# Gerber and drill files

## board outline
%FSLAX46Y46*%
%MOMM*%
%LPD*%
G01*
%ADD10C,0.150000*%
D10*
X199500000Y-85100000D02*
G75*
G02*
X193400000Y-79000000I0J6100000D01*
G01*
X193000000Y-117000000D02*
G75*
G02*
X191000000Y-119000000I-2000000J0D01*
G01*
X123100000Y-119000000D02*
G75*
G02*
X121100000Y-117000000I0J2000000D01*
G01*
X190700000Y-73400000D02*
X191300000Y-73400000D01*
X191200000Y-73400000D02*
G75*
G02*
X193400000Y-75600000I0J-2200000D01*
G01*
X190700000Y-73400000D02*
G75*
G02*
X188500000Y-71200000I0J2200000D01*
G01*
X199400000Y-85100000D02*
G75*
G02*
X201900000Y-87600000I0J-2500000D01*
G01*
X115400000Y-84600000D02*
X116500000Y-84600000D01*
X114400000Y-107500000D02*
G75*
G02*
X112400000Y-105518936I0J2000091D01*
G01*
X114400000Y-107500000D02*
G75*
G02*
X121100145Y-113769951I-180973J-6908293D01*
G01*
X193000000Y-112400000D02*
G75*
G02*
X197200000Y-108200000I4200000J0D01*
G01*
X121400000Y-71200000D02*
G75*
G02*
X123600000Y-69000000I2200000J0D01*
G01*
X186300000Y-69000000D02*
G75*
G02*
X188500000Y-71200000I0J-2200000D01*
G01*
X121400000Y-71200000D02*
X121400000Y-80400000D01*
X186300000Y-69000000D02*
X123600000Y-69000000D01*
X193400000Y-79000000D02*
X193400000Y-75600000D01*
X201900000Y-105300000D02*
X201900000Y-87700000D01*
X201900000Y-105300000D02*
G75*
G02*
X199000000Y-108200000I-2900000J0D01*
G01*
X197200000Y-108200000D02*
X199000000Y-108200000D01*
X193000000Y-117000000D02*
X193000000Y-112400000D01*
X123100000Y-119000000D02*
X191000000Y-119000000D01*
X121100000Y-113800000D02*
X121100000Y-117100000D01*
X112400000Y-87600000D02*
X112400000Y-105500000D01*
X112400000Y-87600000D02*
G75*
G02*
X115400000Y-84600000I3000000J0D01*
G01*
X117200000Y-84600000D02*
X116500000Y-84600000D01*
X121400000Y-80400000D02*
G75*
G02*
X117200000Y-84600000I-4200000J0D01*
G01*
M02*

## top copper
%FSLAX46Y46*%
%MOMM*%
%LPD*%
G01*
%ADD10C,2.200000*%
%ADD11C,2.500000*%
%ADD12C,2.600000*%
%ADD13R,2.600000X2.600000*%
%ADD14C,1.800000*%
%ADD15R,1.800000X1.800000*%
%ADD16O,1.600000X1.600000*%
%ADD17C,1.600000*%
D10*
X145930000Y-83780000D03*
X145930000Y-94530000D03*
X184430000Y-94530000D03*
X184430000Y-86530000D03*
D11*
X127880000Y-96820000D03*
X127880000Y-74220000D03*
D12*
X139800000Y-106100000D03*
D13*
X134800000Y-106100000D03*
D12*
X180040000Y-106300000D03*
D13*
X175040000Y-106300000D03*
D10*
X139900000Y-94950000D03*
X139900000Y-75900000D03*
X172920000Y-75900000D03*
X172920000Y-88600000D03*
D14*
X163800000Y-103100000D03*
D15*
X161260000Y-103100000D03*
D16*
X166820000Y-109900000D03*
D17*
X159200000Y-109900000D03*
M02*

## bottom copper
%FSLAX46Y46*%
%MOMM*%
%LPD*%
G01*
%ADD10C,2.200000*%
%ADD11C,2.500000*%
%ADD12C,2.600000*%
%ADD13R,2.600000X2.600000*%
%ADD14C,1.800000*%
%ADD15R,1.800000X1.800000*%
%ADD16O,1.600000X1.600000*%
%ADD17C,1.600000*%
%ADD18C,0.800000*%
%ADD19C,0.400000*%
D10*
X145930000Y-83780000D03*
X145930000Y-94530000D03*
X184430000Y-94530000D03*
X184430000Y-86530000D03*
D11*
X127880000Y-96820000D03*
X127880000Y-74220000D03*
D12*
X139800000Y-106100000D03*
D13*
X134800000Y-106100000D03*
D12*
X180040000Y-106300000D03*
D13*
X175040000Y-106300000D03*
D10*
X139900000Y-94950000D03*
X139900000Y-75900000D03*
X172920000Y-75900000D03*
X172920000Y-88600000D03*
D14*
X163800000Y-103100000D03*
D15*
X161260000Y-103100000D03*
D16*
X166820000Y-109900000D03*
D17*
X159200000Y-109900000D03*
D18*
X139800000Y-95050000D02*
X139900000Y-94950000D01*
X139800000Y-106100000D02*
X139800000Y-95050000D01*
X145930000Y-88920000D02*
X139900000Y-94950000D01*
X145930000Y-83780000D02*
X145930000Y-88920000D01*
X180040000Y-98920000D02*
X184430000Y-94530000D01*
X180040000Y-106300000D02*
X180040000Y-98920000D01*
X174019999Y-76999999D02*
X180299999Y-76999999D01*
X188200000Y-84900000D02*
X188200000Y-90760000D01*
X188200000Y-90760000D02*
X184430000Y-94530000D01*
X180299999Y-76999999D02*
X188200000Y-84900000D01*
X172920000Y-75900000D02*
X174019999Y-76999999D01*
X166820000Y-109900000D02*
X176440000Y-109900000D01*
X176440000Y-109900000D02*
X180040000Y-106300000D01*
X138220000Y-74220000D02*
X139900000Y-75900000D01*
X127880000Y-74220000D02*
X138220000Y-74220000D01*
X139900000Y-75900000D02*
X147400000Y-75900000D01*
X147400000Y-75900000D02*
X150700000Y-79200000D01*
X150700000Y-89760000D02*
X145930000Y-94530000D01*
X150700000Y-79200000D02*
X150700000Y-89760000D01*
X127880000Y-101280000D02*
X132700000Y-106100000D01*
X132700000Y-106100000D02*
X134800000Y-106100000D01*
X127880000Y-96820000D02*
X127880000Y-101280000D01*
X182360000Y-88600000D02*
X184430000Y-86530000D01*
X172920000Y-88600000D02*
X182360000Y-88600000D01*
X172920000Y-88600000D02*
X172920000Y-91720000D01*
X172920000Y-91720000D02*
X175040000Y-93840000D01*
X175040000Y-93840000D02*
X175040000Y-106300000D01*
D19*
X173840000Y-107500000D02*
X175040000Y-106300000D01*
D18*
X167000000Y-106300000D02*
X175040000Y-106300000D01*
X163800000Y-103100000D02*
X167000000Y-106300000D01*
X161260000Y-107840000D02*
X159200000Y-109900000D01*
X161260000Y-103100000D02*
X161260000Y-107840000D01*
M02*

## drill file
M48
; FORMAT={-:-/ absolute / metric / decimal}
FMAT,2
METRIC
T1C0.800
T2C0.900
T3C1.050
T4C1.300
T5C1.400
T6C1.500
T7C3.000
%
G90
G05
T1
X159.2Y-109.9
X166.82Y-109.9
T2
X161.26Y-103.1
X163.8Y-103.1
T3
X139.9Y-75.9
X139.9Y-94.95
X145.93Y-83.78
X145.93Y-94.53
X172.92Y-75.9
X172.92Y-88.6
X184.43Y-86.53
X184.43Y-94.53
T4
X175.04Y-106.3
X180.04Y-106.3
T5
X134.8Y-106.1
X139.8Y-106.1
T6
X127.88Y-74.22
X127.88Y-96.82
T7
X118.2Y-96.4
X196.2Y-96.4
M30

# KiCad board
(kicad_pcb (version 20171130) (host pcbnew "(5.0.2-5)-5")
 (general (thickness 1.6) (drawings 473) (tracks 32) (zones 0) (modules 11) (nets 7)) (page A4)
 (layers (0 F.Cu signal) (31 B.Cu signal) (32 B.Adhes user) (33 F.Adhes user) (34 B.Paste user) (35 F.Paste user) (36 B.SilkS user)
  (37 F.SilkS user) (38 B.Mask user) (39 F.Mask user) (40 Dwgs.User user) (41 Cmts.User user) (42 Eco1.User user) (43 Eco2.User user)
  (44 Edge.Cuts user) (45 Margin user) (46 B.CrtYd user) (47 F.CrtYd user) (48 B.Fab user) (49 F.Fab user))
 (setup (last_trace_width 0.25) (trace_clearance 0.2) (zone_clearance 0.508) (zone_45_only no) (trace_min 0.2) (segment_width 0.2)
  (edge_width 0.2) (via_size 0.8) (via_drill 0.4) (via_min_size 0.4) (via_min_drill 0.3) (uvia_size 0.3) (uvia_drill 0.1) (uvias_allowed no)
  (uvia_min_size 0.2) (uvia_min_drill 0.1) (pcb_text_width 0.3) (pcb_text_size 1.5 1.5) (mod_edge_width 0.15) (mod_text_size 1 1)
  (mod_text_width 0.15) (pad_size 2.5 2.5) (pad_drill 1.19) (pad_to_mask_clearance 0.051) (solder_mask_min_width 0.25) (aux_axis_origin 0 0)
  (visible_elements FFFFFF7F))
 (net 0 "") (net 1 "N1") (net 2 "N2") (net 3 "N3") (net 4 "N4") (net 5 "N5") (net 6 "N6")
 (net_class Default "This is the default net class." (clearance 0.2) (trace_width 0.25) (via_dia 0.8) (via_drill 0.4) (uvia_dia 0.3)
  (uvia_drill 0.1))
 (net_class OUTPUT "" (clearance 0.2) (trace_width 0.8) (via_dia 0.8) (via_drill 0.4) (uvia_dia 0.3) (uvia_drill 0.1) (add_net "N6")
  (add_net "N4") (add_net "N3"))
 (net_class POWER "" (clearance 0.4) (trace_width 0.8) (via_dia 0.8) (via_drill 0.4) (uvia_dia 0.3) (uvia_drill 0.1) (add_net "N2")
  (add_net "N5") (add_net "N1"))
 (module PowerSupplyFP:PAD (layer F.Cu) (at 196.2 96.4)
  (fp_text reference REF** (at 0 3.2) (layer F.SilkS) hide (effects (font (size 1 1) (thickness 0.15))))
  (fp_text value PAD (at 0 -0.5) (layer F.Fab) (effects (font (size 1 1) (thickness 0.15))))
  (pad "" np_thru_hole circle (at 0 0) (size 3 3) (drill 3) (layers *.Cu *.Mask)))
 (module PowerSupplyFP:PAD (layer F.Cu) (at 118.2 96.4)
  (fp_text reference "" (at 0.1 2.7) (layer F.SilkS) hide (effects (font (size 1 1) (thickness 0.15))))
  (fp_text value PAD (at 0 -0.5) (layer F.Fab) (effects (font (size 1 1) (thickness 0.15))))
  (pad "" np_thru_hole circle (at 0 0) (size 3 3) (drill 3) (layers *.Cu *.Mask)))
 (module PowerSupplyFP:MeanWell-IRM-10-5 (layer F.Cu) (at 142.33 97.98)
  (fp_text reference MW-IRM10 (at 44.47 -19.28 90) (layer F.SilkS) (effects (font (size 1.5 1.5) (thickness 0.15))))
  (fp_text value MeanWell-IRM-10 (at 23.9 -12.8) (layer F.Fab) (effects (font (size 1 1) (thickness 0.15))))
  (pad 1 thru_hole circle (at 3.6 -14.2) (size 2.2 2.2) (drill 1.05) (layers *.Cu *.Mask) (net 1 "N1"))
  (pad 2 thru_hole circle (at 3.6 -3.45) (size 2.2 2.2) (drill 1.05) (layers *.Cu *.Mask) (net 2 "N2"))
  (pad 3 thru_hole circle (at 42.1 -3.45) (size 2.2 2.2) (drill 1.05) (layers *.Cu *.Mask) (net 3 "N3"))
  (pad 4 thru_hole circle (at 42.1 -11.45) (size 2.2 2.2) (drill 1.05) (layers *.Cu *.Mask) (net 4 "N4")))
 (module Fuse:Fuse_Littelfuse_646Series (layer F.Cu) (at 127.88 74.22 270)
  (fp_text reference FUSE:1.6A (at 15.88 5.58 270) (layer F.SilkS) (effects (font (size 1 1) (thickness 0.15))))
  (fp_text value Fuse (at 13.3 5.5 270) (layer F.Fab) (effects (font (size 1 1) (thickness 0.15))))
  (pad 2 thru_hole circle (at 22.6 0 270) (size 2.5 2.5) (drill 1.5) (layers *.Cu *.Mask) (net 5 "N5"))
  (pad 1 thru_hole circle (at 0 0 270) (size 2.5 2.5) (drill 1.5) (layers *.Cu *.Mask) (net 2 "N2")))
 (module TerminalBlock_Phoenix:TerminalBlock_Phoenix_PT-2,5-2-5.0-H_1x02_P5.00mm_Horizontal (layer F.Cu) (at 134.8 106.1)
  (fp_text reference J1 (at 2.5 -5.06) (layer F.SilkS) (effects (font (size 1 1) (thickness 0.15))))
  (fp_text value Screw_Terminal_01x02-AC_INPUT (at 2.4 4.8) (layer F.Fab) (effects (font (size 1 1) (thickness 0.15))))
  (pad 2 thru_hole circle (at 5 0) (size 2.6 2.6) (drill 1.4) (layers *.Cu *.Mask) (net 1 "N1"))
  (pad 1 thru_hole rect (at 0 0) (size 2.6 2.6) (drill 1.4) (layers *.Cu *.Mask) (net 5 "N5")))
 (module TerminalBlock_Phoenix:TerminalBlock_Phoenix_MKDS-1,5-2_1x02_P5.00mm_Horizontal (layer F.Cu) (at 175.04 106.3)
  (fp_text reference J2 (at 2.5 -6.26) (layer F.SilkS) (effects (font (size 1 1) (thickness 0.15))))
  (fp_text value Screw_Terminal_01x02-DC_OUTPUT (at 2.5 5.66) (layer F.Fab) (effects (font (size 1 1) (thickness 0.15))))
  (pad 2 thru_hole circle (at 5 0) (size 2.6 2.6) (drill 1.3) (layers *.Cu *.Mask) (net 3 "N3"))
  (pad 1 thru_hole rect (at 0 0) (size 2.6 2.6) (drill 1.3) (layers *.Cu *.Mask) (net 4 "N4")))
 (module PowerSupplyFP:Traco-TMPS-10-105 (layer F.Cu) (at 137.36 98.76)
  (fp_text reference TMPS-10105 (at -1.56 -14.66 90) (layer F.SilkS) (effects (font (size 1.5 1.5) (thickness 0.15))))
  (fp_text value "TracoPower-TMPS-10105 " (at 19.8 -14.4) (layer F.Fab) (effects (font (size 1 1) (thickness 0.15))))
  (pad 1 thru_hole circle (at 2.54 -3.81) (size 2.2 2.2) (drill 1.05) (layers *.Cu *.Mask) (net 1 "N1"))
  (pad 2 thru_hole circle (at 2.54 -22.86) (size 2.2 2.2) (drill 1.05) (layers *.Cu *.Mask) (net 2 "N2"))
  (pad 3 thru_hole circle (at 35.56 -22.86) (size 2.2 2.2) (drill 1.05) (layers *.Cu *.Mask) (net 3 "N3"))
  (pad 4 thru_hole circle (at 35.56 -10.16) (size 2.2 2.2) (drill 1.05) (layers *.Cu *.Mask) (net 4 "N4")))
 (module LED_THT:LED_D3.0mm (layer F.Cu) (at 161.26 103.1)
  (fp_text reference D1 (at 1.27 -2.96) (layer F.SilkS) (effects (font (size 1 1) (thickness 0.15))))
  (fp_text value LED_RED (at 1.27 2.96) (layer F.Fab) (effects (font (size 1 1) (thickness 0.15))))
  (pad 2 thru_hole circle (at 2.54 0) (size 1.8 1.8) (drill 0.9) (layers *.Cu *.Mask) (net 4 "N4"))
  (pad 1 thru_hole rect (at 0 0) (size 1.8 1.8) (drill 0.9) (layers *.Cu *.Mask) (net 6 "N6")))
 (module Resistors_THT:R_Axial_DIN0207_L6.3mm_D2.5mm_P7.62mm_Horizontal (layer F.Cu) (at 159.2 109.9)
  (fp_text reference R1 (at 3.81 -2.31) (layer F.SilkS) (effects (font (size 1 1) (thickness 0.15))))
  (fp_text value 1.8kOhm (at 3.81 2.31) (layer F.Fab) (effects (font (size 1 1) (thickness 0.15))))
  (pad 2 thru_hole oval (at 7.62 0) (size 1.6 1.6) (drill 0.8) (layers *.Cu *.Mask) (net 3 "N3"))
  (pad 1 thru_hole circle (at 0 0) (size 1.6 1.6) (drill 0.8) (layers *.Cu *.Mask) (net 6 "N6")))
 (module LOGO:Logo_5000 (layer F.Cu) (at 141.9 115)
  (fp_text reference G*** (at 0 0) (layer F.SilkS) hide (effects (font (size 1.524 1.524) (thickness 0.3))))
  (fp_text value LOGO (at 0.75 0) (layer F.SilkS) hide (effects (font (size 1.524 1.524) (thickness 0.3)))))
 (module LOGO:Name (layer F.Cu) (at 130.1 115.3)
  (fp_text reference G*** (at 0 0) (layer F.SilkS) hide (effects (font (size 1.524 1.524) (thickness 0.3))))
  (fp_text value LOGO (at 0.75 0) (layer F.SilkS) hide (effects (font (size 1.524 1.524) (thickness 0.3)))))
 (gr_arc (start 199.5 79) (end 193.4 79) (angle -90) (layer Edge.Cuts) (width 0.15))
 (gr_arc (start 191 117) (end 191 119) (angle -90) (layer Edge.Cuts) (width 0.15))
 (gr_arc (start 123.1 117) (end 121.1 117) (angle -90) (layer Edge.Cuts) (width 0.15))
 (gr_line (start 190.7 73.4) (end 191.3 73.4) (layer Edge.Cuts) (width 0.15))
 (gr_arc (start 191.2 75.6) (end 193.4 75.6) (angle -90) (layer Edge.Cuts) (width 0.15))
 (gr_arc (start 190.7 71.2) (end 188.5 71.2) (angle -90) (layer Edge.Cuts) (width 0.15))
 (gr_arc (start 199.4 87.6) (end 201.9 87.6) (angle -90) (layer Edge.Cuts) (width 0.15))
 (gr_line (start 115.4 84.6) (end 116.5 84.6) (layer Edge.Cuts) (width 0.15))
 (gr_arc (start 114.4 105.499909) (end 112.4 105.518936) (angle -89.45493305) (layer Edge.Cuts) (width 0.15))
 (gr_arc (start 114.219027 114.408293) (end 114.4 107.5) (angle 83.19939526) (layer Edge.Cuts) (width 0.15))
 (gr_arc (start 197.2 112.4) (end 197.2 108.2) (angle -90) (layer Edge.Cuts) (width 0.15))
 (gr_arc (start 123.6 71.2) (end 123.6 69) (angle -90) (layer Edge.Cuts) (width 0.15))
 (gr_arc (start 186.3 71.2) (end 188.5 71.2) (angle -90) (layer Edge.Cuts) (width 0.15))
 (gr_line (start 121.4 71.2) (end 121.4 80.4) (layer Edge.Cuts) (width 0.15))
 (gr_line (start 186.3 69) (end 123.6 69) (layer Edge.Cuts) (width 0.15))
 (gr_line (start 193.4 79) (end 193.4 75.6) (layer Edge.Cuts) (width 0.15))
 (gr_line (start 201.9 105.3) (end 201.9 87.7) (layer Edge.Cuts) (width 0.15))
 (gr_arc (start 199 105.3) (end 199 108.2) (angle -90) (layer Edge.Cuts) (width 0.15))
 (gr_line (start 197.2 108.2) (end 199 108.2) (layer Edge.Cuts) (width 0.15))
 (gr_line (start 193 117) (end 193 112.4) (layer Edge.Cuts) (width 0.15))
 (gr_line (start 123.1 119) (end 191 119) (layer Edge.Cuts) (width 0.15))
 (gr_line (start 121.1 113.8) (end 121.1 117.1) (layer Edge.Cuts) (width 0.15))
 (gr_line (start 112.4 87.6) (end 112.4 105.5) (layer Edge.Cuts) (width 0.15))
 (gr_arc (start 115.4 87.6) (end 115.4 84.6) (angle -90) (layer Edge.Cuts) (width 0.15))
 (gr_line (start 117.2 84.6) (end 116.5 84.6) (layer Edge.Cuts) (width 0.15))
 (gr_arc (start 117.2 80.4) (end 117.2 84.6) (angle -90) (layer Edge.Cuts) (width 0.15))
 (segment (start 139.8 95.05) (end 139.9 94.95) (width 0.8) (layer B.Cu) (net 1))
 (segment (start 139.8 106.1) (end 139.8 95.05) (width 0.8) (layer B.Cu) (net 1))
 (segment (start 145.93 88.92) (end 139.9 94.95) (width 0.8) (layer B.Cu) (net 1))
 (segment (start 145.93 83.78) (end 145.93 88.92) (width 0.8) (layer B.Cu) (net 1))
 (segment (start 180.04 98.92) (end 184.43 94.53) (width 0.8) (layer B.Cu) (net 3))
 (segment (start 180.04 106.3) (end 180.04 98.92) (width 0.8) (layer B.Cu) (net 3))
 (segment (start 174.019999 76.999999) (end 180.299999 76.999999) (width 0.8) (layer B.Cu) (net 3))
 (segment (start 188.2 84.9) (end 188.2 90.76) (width 0.8) (layer B.Cu) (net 3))
 (segment (start 188.2 90.76) (end 184.43 94.53) (width 0.8) (layer B.Cu) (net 3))
 (segment (start 180.299999 76.999999) (end 188.2 84.9) (width 0.8) (layer B.Cu) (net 3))
 (segment (start 172.92 75.9) (end 174.019999 76.999999) (width 0.8) (layer B.Cu) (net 3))
 (segment (start 166.82 109.9) (end 176.44 109.9) (width 0.8) (layer B.Cu) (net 3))
 (segment (start 176.44 109.9) (end 180.04 106.3) (width 0.8) (layer B.Cu) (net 3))
 (segment (start 138.22 74.22) (end 139.9 75.9) (width 0.8) (layer B.Cu) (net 2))
 (segment (start 127.88 74.22) (end 138.22 74.22) (width 0.8) (layer B.Cu) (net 2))
 (segment (start 139.9 75.9) (end 147.4 75.9) (width 0.8) (layer B.Cu) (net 2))
 (segment (start 147.4 75.9) (end 150.7 79.2) (width 0.8) (layer B.Cu) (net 2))
 (segment (start 150.7 89.76) (end 145.93 94.53) (width 0.8) (layer B.Cu) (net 2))
 (segment (start 150.7 79.2) (end 150.7 89.76) (width 0.8) (layer B.Cu) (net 2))
 (segment (start 127.88 101.28) (end 132.7 106.1) (width 0.8) (layer B.Cu) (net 5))
 (segment (start 132.7 106.1) (end 134.8 106.1) (width 0.8) (layer B.Cu) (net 5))
 (segment (start 127.88 96.82) (end 127.88 101.28) (width 0.8) (layer B.Cu) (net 5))
 (segment (start 182.36 88.6) (end 184.43 86.53) (width 0.8) (layer B.Cu) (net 4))
 (segment (start 172.92 88.6) (end 182.36 88.6) (width 0.8) (layer B.Cu) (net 4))
 (segment (start 172.92 88.6) (end 172.92 91.72) (width 0.8) (layer B.Cu) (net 4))
 (segment (start 172.92 91.72) (end 175.04 93.84) (width 0.8) (layer B.Cu) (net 4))
 (segment (start 175.04 93.84) (end 175.04 106.3) (width 0.8) (layer B.Cu) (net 4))
 (segment (start 173.84 107.5) (end 175.04 106.3) (width 0.4) (layer B.Cu) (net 4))
 (segment (start 167 106.3) (end 175.04 106.3) (width 0.8) (layer B.Cu) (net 4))
 (segment (start 163.8 103.1) (end 167 106.3) (width 0.8) (layer B.Cu) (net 4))
 (segment (start 161.26 107.84) (end 159.2 109.9) (width 0.8) (layer B.Cu) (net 6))
 (segment (start 161.26 103.1) (end 161.26 107.84) (width 0.8) (layer B.Cu) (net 6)))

